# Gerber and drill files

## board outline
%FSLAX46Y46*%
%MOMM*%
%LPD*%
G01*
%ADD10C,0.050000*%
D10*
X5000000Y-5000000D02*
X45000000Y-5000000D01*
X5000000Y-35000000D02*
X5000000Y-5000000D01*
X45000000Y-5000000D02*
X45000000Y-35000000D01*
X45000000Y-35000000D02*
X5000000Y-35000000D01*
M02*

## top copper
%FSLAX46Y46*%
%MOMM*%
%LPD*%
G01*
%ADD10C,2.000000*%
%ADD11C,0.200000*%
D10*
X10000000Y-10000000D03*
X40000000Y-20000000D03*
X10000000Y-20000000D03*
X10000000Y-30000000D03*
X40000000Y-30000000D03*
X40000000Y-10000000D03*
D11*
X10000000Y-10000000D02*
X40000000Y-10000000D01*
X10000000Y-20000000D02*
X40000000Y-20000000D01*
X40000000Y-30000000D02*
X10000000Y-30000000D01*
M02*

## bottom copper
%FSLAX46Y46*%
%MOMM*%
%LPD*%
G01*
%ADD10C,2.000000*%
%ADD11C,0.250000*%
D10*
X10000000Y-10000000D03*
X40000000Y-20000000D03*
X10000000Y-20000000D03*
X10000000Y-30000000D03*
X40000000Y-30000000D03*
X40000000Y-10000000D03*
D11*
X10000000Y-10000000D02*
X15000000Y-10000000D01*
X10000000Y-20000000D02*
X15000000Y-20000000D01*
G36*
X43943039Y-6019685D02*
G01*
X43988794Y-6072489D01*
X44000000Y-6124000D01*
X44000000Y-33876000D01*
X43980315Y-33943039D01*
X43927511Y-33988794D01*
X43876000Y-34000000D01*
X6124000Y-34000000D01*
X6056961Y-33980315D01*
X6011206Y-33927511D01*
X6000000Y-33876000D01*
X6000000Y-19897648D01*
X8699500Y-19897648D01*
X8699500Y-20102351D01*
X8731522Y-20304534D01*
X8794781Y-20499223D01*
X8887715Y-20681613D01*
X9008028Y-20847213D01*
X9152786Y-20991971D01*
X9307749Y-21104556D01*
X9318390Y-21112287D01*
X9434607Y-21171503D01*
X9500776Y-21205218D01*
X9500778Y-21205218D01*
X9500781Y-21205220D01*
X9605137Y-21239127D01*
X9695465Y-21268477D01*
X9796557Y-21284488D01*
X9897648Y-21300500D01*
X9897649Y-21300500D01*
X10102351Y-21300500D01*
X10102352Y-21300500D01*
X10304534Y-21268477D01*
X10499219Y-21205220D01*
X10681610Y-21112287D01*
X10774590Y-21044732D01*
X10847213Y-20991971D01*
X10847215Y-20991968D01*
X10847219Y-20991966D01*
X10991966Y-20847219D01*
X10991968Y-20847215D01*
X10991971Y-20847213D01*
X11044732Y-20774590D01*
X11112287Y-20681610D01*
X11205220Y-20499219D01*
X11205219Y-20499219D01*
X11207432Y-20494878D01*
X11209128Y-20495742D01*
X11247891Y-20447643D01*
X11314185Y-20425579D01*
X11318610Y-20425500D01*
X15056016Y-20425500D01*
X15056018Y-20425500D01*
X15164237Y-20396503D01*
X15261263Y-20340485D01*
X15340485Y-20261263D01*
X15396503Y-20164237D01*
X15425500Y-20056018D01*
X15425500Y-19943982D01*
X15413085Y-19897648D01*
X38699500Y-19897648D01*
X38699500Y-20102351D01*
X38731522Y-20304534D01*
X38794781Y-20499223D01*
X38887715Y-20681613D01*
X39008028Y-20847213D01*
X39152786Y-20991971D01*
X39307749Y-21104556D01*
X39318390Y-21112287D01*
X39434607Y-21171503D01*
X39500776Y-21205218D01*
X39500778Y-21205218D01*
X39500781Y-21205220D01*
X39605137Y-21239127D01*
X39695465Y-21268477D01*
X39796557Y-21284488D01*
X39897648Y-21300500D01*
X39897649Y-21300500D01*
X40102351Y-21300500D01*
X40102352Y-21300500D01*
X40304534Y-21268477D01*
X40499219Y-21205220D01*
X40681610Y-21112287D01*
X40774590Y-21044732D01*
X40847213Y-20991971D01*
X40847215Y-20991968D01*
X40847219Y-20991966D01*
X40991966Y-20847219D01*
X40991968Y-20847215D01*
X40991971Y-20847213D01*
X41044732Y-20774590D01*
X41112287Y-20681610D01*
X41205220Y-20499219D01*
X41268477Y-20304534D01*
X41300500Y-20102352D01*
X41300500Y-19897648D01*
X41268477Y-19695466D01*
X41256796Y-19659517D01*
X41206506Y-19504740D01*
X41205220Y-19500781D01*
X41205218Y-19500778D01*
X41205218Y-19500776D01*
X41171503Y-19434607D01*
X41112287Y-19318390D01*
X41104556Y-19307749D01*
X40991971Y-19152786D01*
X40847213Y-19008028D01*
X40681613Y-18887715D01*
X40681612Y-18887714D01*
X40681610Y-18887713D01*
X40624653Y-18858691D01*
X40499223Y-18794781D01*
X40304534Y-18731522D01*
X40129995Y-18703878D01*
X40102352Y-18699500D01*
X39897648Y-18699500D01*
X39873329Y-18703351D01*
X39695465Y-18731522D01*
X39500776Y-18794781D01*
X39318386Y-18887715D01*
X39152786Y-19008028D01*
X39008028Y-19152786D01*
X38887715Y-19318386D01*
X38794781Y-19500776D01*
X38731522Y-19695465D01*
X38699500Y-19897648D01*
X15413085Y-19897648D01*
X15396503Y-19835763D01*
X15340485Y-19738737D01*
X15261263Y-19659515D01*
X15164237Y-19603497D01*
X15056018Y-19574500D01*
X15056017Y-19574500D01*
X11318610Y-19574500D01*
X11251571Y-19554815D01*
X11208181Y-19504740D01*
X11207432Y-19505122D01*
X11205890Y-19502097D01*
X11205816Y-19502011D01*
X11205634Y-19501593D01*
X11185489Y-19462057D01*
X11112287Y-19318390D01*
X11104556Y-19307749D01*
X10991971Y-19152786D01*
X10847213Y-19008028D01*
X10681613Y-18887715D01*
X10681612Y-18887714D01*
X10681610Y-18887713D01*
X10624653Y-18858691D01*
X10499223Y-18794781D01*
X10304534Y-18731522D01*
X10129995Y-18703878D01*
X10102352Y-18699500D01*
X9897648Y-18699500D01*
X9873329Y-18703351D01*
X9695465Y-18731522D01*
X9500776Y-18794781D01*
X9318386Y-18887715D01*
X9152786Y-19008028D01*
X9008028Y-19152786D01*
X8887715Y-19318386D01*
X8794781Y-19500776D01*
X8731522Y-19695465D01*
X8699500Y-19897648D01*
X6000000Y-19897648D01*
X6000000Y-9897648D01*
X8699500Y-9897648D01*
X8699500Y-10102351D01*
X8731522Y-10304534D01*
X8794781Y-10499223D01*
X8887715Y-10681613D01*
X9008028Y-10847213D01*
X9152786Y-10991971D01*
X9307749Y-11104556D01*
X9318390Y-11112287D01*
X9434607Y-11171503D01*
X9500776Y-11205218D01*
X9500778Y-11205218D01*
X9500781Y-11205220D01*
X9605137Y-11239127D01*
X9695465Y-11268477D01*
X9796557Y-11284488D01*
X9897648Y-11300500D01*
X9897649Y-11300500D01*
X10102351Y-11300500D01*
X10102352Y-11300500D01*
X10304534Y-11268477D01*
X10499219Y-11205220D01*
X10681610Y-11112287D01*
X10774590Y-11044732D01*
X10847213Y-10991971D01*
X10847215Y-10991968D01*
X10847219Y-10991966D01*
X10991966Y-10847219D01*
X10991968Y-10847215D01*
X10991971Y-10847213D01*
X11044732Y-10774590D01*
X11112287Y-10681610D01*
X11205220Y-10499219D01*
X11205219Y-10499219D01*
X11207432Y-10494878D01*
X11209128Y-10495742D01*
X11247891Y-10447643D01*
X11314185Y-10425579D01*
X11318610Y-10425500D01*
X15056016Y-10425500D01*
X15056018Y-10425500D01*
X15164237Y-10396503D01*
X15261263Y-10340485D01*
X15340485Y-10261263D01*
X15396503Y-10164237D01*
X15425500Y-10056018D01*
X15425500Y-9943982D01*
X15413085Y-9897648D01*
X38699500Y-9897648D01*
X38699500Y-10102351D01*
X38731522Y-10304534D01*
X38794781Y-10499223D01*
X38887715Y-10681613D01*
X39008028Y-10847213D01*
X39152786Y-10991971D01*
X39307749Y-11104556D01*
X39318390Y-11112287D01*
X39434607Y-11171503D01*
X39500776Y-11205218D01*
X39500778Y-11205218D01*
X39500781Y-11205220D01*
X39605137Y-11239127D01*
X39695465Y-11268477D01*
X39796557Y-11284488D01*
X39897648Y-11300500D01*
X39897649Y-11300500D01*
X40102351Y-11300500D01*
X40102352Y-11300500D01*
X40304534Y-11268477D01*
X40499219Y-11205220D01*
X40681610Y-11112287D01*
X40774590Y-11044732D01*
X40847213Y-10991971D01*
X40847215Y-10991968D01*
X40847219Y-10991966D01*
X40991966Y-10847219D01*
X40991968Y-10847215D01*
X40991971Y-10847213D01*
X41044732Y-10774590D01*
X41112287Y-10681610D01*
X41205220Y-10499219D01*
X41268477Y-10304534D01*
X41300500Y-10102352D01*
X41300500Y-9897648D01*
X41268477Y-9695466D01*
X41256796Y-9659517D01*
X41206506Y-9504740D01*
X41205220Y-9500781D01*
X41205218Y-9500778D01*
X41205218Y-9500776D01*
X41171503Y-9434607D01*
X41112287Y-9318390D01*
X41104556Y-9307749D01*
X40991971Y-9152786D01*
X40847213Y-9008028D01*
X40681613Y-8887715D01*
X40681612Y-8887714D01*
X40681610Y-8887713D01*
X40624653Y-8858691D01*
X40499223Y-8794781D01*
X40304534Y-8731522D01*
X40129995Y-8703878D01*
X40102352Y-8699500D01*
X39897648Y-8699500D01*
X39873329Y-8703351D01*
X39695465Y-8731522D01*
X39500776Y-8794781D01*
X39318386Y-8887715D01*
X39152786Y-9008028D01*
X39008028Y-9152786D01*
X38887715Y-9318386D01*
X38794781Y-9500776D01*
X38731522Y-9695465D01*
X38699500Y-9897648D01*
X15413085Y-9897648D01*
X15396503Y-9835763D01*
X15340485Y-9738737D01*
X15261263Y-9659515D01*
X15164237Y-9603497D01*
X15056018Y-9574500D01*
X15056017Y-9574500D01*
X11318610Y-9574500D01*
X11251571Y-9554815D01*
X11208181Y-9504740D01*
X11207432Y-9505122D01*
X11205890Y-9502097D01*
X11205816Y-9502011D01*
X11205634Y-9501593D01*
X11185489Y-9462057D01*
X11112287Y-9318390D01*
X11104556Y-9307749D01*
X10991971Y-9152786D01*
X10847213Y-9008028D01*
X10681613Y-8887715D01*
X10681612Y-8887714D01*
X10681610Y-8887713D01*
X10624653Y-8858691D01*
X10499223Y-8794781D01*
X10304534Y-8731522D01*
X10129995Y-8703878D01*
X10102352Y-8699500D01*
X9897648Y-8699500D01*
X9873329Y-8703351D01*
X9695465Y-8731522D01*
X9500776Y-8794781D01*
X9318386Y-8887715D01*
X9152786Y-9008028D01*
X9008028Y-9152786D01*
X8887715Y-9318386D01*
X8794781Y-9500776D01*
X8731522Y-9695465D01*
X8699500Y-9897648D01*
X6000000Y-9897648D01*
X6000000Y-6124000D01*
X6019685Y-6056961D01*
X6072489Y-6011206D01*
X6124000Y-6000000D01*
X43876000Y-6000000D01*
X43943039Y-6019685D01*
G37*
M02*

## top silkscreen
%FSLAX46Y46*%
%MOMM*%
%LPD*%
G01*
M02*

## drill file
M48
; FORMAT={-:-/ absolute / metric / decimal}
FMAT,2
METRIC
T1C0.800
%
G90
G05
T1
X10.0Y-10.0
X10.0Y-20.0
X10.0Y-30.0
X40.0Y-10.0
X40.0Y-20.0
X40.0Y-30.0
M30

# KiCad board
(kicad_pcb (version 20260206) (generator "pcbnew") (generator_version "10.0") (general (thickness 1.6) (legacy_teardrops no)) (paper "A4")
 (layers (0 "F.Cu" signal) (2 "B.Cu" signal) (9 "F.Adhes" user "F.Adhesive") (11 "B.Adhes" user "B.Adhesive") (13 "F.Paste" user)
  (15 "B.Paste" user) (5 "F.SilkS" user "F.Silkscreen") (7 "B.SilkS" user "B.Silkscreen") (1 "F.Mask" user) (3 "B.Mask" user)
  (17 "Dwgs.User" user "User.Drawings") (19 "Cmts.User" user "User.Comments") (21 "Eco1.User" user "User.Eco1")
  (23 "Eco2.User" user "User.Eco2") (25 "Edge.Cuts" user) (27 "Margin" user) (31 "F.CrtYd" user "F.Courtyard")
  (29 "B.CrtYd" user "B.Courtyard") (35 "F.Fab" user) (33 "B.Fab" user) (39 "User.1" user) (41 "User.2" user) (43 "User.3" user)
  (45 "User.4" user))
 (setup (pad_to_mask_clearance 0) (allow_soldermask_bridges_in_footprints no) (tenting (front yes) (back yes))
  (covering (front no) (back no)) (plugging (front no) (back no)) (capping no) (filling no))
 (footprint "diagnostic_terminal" (layer "F.Cu") (at 10 10)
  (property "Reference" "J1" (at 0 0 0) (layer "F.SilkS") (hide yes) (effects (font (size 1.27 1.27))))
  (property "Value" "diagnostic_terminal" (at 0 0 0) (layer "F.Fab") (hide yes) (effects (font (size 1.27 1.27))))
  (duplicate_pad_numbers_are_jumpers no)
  (pad "1" thru_hole circle (at 0 0) (size 2 2) (drill 0.8) (layers "*.Cu") (remove_unused_layers no) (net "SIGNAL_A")))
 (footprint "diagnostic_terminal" (layer "F.Cu") (at 40 20)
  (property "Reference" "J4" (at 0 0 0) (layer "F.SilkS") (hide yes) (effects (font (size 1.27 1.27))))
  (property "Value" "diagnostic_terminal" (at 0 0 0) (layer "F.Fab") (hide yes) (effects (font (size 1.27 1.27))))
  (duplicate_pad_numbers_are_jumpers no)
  (pad "1" thru_hole circle (at 0 0) (size 2 2) (drill 0.8) (layers "*.Cu") (remove_unused_layers no) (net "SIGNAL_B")))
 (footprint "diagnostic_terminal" (layer "F.Cu") (at 10 20)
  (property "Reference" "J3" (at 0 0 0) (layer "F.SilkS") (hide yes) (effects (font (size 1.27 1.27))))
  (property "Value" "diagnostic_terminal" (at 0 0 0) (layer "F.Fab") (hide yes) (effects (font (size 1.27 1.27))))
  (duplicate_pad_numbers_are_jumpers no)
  (pad "1" thru_hole circle (at 0 0) (size 2 2) (drill 0.8) (layers "*.Cu") (remove_unused_layers no) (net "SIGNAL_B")))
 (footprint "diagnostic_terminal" (layer "F.Cu") (at 10 30)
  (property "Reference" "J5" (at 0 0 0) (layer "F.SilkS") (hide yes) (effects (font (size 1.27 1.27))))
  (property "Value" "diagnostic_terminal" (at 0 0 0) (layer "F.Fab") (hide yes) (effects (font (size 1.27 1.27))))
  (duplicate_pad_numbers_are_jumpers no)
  (pad "1" thru_hole circle (at 0 0) (size 2 2) (drill 0.8) (layers "*.Cu") (remove_unused_layers no) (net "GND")))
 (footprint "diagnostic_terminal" (layer "F.Cu") (at 40 30)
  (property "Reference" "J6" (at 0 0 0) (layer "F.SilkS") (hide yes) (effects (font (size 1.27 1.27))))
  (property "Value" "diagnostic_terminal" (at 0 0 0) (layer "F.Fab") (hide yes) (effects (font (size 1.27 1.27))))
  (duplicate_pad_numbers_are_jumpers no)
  (pad "1" thru_hole circle (at 0 0) (size 2 2) (drill 0.8) (layers "*.Cu") (remove_unused_layers no) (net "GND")))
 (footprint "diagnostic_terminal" (layer "F.Cu") (at 40 10)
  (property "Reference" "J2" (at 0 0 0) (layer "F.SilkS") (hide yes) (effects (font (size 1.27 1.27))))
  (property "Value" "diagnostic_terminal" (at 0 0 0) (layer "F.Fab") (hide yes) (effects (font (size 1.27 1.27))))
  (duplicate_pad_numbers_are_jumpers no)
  (pad "1" thru_hole circle (at 0 0) (size 2 2) (drill 0.8) (layers "*.Cu") (remove_unused_layers no) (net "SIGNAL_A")))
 (gr_line (start 5 5) (end 45 5) (stroke (width 0.05) (type default)) (layer "Edge.Cuts"))
 (gr_line (start 5 35) (end 5 5) (stroke (width 0.05) (type default)) (layer "Edge.Cuts"))
 (gr_line (start 45 5) (end 45 35) (stroke (width 0.05) (type default)) (layer "Edge.Cuts"))
 (gr_line (start 45 35) (end 5 35) (stroke (width 0.05) (type default)) (layer "Edge.Cuts"))
 (segment (start 10 10) (end 40 10) (width 0.2) (layer "F.Cu") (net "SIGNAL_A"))
 (segment (start 10 10) (end 15 10) (width 0.25) (layer "B.Cu") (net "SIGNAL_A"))
 (segment (start 10 20) (end 40 20) (width 0.2) (layer "F.Cu") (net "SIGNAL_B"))
 (segment (start 10 20) (end 15 20) (width 0.25) (layer "B.Cu") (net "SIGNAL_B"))
 (segment (start 40 30) (end 10 30) (width 0.2) (layer "F.Cu") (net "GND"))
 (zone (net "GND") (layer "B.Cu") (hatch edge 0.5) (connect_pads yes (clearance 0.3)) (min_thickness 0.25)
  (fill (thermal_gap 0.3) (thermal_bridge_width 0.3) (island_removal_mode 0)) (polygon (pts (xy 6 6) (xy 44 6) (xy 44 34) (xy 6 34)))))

